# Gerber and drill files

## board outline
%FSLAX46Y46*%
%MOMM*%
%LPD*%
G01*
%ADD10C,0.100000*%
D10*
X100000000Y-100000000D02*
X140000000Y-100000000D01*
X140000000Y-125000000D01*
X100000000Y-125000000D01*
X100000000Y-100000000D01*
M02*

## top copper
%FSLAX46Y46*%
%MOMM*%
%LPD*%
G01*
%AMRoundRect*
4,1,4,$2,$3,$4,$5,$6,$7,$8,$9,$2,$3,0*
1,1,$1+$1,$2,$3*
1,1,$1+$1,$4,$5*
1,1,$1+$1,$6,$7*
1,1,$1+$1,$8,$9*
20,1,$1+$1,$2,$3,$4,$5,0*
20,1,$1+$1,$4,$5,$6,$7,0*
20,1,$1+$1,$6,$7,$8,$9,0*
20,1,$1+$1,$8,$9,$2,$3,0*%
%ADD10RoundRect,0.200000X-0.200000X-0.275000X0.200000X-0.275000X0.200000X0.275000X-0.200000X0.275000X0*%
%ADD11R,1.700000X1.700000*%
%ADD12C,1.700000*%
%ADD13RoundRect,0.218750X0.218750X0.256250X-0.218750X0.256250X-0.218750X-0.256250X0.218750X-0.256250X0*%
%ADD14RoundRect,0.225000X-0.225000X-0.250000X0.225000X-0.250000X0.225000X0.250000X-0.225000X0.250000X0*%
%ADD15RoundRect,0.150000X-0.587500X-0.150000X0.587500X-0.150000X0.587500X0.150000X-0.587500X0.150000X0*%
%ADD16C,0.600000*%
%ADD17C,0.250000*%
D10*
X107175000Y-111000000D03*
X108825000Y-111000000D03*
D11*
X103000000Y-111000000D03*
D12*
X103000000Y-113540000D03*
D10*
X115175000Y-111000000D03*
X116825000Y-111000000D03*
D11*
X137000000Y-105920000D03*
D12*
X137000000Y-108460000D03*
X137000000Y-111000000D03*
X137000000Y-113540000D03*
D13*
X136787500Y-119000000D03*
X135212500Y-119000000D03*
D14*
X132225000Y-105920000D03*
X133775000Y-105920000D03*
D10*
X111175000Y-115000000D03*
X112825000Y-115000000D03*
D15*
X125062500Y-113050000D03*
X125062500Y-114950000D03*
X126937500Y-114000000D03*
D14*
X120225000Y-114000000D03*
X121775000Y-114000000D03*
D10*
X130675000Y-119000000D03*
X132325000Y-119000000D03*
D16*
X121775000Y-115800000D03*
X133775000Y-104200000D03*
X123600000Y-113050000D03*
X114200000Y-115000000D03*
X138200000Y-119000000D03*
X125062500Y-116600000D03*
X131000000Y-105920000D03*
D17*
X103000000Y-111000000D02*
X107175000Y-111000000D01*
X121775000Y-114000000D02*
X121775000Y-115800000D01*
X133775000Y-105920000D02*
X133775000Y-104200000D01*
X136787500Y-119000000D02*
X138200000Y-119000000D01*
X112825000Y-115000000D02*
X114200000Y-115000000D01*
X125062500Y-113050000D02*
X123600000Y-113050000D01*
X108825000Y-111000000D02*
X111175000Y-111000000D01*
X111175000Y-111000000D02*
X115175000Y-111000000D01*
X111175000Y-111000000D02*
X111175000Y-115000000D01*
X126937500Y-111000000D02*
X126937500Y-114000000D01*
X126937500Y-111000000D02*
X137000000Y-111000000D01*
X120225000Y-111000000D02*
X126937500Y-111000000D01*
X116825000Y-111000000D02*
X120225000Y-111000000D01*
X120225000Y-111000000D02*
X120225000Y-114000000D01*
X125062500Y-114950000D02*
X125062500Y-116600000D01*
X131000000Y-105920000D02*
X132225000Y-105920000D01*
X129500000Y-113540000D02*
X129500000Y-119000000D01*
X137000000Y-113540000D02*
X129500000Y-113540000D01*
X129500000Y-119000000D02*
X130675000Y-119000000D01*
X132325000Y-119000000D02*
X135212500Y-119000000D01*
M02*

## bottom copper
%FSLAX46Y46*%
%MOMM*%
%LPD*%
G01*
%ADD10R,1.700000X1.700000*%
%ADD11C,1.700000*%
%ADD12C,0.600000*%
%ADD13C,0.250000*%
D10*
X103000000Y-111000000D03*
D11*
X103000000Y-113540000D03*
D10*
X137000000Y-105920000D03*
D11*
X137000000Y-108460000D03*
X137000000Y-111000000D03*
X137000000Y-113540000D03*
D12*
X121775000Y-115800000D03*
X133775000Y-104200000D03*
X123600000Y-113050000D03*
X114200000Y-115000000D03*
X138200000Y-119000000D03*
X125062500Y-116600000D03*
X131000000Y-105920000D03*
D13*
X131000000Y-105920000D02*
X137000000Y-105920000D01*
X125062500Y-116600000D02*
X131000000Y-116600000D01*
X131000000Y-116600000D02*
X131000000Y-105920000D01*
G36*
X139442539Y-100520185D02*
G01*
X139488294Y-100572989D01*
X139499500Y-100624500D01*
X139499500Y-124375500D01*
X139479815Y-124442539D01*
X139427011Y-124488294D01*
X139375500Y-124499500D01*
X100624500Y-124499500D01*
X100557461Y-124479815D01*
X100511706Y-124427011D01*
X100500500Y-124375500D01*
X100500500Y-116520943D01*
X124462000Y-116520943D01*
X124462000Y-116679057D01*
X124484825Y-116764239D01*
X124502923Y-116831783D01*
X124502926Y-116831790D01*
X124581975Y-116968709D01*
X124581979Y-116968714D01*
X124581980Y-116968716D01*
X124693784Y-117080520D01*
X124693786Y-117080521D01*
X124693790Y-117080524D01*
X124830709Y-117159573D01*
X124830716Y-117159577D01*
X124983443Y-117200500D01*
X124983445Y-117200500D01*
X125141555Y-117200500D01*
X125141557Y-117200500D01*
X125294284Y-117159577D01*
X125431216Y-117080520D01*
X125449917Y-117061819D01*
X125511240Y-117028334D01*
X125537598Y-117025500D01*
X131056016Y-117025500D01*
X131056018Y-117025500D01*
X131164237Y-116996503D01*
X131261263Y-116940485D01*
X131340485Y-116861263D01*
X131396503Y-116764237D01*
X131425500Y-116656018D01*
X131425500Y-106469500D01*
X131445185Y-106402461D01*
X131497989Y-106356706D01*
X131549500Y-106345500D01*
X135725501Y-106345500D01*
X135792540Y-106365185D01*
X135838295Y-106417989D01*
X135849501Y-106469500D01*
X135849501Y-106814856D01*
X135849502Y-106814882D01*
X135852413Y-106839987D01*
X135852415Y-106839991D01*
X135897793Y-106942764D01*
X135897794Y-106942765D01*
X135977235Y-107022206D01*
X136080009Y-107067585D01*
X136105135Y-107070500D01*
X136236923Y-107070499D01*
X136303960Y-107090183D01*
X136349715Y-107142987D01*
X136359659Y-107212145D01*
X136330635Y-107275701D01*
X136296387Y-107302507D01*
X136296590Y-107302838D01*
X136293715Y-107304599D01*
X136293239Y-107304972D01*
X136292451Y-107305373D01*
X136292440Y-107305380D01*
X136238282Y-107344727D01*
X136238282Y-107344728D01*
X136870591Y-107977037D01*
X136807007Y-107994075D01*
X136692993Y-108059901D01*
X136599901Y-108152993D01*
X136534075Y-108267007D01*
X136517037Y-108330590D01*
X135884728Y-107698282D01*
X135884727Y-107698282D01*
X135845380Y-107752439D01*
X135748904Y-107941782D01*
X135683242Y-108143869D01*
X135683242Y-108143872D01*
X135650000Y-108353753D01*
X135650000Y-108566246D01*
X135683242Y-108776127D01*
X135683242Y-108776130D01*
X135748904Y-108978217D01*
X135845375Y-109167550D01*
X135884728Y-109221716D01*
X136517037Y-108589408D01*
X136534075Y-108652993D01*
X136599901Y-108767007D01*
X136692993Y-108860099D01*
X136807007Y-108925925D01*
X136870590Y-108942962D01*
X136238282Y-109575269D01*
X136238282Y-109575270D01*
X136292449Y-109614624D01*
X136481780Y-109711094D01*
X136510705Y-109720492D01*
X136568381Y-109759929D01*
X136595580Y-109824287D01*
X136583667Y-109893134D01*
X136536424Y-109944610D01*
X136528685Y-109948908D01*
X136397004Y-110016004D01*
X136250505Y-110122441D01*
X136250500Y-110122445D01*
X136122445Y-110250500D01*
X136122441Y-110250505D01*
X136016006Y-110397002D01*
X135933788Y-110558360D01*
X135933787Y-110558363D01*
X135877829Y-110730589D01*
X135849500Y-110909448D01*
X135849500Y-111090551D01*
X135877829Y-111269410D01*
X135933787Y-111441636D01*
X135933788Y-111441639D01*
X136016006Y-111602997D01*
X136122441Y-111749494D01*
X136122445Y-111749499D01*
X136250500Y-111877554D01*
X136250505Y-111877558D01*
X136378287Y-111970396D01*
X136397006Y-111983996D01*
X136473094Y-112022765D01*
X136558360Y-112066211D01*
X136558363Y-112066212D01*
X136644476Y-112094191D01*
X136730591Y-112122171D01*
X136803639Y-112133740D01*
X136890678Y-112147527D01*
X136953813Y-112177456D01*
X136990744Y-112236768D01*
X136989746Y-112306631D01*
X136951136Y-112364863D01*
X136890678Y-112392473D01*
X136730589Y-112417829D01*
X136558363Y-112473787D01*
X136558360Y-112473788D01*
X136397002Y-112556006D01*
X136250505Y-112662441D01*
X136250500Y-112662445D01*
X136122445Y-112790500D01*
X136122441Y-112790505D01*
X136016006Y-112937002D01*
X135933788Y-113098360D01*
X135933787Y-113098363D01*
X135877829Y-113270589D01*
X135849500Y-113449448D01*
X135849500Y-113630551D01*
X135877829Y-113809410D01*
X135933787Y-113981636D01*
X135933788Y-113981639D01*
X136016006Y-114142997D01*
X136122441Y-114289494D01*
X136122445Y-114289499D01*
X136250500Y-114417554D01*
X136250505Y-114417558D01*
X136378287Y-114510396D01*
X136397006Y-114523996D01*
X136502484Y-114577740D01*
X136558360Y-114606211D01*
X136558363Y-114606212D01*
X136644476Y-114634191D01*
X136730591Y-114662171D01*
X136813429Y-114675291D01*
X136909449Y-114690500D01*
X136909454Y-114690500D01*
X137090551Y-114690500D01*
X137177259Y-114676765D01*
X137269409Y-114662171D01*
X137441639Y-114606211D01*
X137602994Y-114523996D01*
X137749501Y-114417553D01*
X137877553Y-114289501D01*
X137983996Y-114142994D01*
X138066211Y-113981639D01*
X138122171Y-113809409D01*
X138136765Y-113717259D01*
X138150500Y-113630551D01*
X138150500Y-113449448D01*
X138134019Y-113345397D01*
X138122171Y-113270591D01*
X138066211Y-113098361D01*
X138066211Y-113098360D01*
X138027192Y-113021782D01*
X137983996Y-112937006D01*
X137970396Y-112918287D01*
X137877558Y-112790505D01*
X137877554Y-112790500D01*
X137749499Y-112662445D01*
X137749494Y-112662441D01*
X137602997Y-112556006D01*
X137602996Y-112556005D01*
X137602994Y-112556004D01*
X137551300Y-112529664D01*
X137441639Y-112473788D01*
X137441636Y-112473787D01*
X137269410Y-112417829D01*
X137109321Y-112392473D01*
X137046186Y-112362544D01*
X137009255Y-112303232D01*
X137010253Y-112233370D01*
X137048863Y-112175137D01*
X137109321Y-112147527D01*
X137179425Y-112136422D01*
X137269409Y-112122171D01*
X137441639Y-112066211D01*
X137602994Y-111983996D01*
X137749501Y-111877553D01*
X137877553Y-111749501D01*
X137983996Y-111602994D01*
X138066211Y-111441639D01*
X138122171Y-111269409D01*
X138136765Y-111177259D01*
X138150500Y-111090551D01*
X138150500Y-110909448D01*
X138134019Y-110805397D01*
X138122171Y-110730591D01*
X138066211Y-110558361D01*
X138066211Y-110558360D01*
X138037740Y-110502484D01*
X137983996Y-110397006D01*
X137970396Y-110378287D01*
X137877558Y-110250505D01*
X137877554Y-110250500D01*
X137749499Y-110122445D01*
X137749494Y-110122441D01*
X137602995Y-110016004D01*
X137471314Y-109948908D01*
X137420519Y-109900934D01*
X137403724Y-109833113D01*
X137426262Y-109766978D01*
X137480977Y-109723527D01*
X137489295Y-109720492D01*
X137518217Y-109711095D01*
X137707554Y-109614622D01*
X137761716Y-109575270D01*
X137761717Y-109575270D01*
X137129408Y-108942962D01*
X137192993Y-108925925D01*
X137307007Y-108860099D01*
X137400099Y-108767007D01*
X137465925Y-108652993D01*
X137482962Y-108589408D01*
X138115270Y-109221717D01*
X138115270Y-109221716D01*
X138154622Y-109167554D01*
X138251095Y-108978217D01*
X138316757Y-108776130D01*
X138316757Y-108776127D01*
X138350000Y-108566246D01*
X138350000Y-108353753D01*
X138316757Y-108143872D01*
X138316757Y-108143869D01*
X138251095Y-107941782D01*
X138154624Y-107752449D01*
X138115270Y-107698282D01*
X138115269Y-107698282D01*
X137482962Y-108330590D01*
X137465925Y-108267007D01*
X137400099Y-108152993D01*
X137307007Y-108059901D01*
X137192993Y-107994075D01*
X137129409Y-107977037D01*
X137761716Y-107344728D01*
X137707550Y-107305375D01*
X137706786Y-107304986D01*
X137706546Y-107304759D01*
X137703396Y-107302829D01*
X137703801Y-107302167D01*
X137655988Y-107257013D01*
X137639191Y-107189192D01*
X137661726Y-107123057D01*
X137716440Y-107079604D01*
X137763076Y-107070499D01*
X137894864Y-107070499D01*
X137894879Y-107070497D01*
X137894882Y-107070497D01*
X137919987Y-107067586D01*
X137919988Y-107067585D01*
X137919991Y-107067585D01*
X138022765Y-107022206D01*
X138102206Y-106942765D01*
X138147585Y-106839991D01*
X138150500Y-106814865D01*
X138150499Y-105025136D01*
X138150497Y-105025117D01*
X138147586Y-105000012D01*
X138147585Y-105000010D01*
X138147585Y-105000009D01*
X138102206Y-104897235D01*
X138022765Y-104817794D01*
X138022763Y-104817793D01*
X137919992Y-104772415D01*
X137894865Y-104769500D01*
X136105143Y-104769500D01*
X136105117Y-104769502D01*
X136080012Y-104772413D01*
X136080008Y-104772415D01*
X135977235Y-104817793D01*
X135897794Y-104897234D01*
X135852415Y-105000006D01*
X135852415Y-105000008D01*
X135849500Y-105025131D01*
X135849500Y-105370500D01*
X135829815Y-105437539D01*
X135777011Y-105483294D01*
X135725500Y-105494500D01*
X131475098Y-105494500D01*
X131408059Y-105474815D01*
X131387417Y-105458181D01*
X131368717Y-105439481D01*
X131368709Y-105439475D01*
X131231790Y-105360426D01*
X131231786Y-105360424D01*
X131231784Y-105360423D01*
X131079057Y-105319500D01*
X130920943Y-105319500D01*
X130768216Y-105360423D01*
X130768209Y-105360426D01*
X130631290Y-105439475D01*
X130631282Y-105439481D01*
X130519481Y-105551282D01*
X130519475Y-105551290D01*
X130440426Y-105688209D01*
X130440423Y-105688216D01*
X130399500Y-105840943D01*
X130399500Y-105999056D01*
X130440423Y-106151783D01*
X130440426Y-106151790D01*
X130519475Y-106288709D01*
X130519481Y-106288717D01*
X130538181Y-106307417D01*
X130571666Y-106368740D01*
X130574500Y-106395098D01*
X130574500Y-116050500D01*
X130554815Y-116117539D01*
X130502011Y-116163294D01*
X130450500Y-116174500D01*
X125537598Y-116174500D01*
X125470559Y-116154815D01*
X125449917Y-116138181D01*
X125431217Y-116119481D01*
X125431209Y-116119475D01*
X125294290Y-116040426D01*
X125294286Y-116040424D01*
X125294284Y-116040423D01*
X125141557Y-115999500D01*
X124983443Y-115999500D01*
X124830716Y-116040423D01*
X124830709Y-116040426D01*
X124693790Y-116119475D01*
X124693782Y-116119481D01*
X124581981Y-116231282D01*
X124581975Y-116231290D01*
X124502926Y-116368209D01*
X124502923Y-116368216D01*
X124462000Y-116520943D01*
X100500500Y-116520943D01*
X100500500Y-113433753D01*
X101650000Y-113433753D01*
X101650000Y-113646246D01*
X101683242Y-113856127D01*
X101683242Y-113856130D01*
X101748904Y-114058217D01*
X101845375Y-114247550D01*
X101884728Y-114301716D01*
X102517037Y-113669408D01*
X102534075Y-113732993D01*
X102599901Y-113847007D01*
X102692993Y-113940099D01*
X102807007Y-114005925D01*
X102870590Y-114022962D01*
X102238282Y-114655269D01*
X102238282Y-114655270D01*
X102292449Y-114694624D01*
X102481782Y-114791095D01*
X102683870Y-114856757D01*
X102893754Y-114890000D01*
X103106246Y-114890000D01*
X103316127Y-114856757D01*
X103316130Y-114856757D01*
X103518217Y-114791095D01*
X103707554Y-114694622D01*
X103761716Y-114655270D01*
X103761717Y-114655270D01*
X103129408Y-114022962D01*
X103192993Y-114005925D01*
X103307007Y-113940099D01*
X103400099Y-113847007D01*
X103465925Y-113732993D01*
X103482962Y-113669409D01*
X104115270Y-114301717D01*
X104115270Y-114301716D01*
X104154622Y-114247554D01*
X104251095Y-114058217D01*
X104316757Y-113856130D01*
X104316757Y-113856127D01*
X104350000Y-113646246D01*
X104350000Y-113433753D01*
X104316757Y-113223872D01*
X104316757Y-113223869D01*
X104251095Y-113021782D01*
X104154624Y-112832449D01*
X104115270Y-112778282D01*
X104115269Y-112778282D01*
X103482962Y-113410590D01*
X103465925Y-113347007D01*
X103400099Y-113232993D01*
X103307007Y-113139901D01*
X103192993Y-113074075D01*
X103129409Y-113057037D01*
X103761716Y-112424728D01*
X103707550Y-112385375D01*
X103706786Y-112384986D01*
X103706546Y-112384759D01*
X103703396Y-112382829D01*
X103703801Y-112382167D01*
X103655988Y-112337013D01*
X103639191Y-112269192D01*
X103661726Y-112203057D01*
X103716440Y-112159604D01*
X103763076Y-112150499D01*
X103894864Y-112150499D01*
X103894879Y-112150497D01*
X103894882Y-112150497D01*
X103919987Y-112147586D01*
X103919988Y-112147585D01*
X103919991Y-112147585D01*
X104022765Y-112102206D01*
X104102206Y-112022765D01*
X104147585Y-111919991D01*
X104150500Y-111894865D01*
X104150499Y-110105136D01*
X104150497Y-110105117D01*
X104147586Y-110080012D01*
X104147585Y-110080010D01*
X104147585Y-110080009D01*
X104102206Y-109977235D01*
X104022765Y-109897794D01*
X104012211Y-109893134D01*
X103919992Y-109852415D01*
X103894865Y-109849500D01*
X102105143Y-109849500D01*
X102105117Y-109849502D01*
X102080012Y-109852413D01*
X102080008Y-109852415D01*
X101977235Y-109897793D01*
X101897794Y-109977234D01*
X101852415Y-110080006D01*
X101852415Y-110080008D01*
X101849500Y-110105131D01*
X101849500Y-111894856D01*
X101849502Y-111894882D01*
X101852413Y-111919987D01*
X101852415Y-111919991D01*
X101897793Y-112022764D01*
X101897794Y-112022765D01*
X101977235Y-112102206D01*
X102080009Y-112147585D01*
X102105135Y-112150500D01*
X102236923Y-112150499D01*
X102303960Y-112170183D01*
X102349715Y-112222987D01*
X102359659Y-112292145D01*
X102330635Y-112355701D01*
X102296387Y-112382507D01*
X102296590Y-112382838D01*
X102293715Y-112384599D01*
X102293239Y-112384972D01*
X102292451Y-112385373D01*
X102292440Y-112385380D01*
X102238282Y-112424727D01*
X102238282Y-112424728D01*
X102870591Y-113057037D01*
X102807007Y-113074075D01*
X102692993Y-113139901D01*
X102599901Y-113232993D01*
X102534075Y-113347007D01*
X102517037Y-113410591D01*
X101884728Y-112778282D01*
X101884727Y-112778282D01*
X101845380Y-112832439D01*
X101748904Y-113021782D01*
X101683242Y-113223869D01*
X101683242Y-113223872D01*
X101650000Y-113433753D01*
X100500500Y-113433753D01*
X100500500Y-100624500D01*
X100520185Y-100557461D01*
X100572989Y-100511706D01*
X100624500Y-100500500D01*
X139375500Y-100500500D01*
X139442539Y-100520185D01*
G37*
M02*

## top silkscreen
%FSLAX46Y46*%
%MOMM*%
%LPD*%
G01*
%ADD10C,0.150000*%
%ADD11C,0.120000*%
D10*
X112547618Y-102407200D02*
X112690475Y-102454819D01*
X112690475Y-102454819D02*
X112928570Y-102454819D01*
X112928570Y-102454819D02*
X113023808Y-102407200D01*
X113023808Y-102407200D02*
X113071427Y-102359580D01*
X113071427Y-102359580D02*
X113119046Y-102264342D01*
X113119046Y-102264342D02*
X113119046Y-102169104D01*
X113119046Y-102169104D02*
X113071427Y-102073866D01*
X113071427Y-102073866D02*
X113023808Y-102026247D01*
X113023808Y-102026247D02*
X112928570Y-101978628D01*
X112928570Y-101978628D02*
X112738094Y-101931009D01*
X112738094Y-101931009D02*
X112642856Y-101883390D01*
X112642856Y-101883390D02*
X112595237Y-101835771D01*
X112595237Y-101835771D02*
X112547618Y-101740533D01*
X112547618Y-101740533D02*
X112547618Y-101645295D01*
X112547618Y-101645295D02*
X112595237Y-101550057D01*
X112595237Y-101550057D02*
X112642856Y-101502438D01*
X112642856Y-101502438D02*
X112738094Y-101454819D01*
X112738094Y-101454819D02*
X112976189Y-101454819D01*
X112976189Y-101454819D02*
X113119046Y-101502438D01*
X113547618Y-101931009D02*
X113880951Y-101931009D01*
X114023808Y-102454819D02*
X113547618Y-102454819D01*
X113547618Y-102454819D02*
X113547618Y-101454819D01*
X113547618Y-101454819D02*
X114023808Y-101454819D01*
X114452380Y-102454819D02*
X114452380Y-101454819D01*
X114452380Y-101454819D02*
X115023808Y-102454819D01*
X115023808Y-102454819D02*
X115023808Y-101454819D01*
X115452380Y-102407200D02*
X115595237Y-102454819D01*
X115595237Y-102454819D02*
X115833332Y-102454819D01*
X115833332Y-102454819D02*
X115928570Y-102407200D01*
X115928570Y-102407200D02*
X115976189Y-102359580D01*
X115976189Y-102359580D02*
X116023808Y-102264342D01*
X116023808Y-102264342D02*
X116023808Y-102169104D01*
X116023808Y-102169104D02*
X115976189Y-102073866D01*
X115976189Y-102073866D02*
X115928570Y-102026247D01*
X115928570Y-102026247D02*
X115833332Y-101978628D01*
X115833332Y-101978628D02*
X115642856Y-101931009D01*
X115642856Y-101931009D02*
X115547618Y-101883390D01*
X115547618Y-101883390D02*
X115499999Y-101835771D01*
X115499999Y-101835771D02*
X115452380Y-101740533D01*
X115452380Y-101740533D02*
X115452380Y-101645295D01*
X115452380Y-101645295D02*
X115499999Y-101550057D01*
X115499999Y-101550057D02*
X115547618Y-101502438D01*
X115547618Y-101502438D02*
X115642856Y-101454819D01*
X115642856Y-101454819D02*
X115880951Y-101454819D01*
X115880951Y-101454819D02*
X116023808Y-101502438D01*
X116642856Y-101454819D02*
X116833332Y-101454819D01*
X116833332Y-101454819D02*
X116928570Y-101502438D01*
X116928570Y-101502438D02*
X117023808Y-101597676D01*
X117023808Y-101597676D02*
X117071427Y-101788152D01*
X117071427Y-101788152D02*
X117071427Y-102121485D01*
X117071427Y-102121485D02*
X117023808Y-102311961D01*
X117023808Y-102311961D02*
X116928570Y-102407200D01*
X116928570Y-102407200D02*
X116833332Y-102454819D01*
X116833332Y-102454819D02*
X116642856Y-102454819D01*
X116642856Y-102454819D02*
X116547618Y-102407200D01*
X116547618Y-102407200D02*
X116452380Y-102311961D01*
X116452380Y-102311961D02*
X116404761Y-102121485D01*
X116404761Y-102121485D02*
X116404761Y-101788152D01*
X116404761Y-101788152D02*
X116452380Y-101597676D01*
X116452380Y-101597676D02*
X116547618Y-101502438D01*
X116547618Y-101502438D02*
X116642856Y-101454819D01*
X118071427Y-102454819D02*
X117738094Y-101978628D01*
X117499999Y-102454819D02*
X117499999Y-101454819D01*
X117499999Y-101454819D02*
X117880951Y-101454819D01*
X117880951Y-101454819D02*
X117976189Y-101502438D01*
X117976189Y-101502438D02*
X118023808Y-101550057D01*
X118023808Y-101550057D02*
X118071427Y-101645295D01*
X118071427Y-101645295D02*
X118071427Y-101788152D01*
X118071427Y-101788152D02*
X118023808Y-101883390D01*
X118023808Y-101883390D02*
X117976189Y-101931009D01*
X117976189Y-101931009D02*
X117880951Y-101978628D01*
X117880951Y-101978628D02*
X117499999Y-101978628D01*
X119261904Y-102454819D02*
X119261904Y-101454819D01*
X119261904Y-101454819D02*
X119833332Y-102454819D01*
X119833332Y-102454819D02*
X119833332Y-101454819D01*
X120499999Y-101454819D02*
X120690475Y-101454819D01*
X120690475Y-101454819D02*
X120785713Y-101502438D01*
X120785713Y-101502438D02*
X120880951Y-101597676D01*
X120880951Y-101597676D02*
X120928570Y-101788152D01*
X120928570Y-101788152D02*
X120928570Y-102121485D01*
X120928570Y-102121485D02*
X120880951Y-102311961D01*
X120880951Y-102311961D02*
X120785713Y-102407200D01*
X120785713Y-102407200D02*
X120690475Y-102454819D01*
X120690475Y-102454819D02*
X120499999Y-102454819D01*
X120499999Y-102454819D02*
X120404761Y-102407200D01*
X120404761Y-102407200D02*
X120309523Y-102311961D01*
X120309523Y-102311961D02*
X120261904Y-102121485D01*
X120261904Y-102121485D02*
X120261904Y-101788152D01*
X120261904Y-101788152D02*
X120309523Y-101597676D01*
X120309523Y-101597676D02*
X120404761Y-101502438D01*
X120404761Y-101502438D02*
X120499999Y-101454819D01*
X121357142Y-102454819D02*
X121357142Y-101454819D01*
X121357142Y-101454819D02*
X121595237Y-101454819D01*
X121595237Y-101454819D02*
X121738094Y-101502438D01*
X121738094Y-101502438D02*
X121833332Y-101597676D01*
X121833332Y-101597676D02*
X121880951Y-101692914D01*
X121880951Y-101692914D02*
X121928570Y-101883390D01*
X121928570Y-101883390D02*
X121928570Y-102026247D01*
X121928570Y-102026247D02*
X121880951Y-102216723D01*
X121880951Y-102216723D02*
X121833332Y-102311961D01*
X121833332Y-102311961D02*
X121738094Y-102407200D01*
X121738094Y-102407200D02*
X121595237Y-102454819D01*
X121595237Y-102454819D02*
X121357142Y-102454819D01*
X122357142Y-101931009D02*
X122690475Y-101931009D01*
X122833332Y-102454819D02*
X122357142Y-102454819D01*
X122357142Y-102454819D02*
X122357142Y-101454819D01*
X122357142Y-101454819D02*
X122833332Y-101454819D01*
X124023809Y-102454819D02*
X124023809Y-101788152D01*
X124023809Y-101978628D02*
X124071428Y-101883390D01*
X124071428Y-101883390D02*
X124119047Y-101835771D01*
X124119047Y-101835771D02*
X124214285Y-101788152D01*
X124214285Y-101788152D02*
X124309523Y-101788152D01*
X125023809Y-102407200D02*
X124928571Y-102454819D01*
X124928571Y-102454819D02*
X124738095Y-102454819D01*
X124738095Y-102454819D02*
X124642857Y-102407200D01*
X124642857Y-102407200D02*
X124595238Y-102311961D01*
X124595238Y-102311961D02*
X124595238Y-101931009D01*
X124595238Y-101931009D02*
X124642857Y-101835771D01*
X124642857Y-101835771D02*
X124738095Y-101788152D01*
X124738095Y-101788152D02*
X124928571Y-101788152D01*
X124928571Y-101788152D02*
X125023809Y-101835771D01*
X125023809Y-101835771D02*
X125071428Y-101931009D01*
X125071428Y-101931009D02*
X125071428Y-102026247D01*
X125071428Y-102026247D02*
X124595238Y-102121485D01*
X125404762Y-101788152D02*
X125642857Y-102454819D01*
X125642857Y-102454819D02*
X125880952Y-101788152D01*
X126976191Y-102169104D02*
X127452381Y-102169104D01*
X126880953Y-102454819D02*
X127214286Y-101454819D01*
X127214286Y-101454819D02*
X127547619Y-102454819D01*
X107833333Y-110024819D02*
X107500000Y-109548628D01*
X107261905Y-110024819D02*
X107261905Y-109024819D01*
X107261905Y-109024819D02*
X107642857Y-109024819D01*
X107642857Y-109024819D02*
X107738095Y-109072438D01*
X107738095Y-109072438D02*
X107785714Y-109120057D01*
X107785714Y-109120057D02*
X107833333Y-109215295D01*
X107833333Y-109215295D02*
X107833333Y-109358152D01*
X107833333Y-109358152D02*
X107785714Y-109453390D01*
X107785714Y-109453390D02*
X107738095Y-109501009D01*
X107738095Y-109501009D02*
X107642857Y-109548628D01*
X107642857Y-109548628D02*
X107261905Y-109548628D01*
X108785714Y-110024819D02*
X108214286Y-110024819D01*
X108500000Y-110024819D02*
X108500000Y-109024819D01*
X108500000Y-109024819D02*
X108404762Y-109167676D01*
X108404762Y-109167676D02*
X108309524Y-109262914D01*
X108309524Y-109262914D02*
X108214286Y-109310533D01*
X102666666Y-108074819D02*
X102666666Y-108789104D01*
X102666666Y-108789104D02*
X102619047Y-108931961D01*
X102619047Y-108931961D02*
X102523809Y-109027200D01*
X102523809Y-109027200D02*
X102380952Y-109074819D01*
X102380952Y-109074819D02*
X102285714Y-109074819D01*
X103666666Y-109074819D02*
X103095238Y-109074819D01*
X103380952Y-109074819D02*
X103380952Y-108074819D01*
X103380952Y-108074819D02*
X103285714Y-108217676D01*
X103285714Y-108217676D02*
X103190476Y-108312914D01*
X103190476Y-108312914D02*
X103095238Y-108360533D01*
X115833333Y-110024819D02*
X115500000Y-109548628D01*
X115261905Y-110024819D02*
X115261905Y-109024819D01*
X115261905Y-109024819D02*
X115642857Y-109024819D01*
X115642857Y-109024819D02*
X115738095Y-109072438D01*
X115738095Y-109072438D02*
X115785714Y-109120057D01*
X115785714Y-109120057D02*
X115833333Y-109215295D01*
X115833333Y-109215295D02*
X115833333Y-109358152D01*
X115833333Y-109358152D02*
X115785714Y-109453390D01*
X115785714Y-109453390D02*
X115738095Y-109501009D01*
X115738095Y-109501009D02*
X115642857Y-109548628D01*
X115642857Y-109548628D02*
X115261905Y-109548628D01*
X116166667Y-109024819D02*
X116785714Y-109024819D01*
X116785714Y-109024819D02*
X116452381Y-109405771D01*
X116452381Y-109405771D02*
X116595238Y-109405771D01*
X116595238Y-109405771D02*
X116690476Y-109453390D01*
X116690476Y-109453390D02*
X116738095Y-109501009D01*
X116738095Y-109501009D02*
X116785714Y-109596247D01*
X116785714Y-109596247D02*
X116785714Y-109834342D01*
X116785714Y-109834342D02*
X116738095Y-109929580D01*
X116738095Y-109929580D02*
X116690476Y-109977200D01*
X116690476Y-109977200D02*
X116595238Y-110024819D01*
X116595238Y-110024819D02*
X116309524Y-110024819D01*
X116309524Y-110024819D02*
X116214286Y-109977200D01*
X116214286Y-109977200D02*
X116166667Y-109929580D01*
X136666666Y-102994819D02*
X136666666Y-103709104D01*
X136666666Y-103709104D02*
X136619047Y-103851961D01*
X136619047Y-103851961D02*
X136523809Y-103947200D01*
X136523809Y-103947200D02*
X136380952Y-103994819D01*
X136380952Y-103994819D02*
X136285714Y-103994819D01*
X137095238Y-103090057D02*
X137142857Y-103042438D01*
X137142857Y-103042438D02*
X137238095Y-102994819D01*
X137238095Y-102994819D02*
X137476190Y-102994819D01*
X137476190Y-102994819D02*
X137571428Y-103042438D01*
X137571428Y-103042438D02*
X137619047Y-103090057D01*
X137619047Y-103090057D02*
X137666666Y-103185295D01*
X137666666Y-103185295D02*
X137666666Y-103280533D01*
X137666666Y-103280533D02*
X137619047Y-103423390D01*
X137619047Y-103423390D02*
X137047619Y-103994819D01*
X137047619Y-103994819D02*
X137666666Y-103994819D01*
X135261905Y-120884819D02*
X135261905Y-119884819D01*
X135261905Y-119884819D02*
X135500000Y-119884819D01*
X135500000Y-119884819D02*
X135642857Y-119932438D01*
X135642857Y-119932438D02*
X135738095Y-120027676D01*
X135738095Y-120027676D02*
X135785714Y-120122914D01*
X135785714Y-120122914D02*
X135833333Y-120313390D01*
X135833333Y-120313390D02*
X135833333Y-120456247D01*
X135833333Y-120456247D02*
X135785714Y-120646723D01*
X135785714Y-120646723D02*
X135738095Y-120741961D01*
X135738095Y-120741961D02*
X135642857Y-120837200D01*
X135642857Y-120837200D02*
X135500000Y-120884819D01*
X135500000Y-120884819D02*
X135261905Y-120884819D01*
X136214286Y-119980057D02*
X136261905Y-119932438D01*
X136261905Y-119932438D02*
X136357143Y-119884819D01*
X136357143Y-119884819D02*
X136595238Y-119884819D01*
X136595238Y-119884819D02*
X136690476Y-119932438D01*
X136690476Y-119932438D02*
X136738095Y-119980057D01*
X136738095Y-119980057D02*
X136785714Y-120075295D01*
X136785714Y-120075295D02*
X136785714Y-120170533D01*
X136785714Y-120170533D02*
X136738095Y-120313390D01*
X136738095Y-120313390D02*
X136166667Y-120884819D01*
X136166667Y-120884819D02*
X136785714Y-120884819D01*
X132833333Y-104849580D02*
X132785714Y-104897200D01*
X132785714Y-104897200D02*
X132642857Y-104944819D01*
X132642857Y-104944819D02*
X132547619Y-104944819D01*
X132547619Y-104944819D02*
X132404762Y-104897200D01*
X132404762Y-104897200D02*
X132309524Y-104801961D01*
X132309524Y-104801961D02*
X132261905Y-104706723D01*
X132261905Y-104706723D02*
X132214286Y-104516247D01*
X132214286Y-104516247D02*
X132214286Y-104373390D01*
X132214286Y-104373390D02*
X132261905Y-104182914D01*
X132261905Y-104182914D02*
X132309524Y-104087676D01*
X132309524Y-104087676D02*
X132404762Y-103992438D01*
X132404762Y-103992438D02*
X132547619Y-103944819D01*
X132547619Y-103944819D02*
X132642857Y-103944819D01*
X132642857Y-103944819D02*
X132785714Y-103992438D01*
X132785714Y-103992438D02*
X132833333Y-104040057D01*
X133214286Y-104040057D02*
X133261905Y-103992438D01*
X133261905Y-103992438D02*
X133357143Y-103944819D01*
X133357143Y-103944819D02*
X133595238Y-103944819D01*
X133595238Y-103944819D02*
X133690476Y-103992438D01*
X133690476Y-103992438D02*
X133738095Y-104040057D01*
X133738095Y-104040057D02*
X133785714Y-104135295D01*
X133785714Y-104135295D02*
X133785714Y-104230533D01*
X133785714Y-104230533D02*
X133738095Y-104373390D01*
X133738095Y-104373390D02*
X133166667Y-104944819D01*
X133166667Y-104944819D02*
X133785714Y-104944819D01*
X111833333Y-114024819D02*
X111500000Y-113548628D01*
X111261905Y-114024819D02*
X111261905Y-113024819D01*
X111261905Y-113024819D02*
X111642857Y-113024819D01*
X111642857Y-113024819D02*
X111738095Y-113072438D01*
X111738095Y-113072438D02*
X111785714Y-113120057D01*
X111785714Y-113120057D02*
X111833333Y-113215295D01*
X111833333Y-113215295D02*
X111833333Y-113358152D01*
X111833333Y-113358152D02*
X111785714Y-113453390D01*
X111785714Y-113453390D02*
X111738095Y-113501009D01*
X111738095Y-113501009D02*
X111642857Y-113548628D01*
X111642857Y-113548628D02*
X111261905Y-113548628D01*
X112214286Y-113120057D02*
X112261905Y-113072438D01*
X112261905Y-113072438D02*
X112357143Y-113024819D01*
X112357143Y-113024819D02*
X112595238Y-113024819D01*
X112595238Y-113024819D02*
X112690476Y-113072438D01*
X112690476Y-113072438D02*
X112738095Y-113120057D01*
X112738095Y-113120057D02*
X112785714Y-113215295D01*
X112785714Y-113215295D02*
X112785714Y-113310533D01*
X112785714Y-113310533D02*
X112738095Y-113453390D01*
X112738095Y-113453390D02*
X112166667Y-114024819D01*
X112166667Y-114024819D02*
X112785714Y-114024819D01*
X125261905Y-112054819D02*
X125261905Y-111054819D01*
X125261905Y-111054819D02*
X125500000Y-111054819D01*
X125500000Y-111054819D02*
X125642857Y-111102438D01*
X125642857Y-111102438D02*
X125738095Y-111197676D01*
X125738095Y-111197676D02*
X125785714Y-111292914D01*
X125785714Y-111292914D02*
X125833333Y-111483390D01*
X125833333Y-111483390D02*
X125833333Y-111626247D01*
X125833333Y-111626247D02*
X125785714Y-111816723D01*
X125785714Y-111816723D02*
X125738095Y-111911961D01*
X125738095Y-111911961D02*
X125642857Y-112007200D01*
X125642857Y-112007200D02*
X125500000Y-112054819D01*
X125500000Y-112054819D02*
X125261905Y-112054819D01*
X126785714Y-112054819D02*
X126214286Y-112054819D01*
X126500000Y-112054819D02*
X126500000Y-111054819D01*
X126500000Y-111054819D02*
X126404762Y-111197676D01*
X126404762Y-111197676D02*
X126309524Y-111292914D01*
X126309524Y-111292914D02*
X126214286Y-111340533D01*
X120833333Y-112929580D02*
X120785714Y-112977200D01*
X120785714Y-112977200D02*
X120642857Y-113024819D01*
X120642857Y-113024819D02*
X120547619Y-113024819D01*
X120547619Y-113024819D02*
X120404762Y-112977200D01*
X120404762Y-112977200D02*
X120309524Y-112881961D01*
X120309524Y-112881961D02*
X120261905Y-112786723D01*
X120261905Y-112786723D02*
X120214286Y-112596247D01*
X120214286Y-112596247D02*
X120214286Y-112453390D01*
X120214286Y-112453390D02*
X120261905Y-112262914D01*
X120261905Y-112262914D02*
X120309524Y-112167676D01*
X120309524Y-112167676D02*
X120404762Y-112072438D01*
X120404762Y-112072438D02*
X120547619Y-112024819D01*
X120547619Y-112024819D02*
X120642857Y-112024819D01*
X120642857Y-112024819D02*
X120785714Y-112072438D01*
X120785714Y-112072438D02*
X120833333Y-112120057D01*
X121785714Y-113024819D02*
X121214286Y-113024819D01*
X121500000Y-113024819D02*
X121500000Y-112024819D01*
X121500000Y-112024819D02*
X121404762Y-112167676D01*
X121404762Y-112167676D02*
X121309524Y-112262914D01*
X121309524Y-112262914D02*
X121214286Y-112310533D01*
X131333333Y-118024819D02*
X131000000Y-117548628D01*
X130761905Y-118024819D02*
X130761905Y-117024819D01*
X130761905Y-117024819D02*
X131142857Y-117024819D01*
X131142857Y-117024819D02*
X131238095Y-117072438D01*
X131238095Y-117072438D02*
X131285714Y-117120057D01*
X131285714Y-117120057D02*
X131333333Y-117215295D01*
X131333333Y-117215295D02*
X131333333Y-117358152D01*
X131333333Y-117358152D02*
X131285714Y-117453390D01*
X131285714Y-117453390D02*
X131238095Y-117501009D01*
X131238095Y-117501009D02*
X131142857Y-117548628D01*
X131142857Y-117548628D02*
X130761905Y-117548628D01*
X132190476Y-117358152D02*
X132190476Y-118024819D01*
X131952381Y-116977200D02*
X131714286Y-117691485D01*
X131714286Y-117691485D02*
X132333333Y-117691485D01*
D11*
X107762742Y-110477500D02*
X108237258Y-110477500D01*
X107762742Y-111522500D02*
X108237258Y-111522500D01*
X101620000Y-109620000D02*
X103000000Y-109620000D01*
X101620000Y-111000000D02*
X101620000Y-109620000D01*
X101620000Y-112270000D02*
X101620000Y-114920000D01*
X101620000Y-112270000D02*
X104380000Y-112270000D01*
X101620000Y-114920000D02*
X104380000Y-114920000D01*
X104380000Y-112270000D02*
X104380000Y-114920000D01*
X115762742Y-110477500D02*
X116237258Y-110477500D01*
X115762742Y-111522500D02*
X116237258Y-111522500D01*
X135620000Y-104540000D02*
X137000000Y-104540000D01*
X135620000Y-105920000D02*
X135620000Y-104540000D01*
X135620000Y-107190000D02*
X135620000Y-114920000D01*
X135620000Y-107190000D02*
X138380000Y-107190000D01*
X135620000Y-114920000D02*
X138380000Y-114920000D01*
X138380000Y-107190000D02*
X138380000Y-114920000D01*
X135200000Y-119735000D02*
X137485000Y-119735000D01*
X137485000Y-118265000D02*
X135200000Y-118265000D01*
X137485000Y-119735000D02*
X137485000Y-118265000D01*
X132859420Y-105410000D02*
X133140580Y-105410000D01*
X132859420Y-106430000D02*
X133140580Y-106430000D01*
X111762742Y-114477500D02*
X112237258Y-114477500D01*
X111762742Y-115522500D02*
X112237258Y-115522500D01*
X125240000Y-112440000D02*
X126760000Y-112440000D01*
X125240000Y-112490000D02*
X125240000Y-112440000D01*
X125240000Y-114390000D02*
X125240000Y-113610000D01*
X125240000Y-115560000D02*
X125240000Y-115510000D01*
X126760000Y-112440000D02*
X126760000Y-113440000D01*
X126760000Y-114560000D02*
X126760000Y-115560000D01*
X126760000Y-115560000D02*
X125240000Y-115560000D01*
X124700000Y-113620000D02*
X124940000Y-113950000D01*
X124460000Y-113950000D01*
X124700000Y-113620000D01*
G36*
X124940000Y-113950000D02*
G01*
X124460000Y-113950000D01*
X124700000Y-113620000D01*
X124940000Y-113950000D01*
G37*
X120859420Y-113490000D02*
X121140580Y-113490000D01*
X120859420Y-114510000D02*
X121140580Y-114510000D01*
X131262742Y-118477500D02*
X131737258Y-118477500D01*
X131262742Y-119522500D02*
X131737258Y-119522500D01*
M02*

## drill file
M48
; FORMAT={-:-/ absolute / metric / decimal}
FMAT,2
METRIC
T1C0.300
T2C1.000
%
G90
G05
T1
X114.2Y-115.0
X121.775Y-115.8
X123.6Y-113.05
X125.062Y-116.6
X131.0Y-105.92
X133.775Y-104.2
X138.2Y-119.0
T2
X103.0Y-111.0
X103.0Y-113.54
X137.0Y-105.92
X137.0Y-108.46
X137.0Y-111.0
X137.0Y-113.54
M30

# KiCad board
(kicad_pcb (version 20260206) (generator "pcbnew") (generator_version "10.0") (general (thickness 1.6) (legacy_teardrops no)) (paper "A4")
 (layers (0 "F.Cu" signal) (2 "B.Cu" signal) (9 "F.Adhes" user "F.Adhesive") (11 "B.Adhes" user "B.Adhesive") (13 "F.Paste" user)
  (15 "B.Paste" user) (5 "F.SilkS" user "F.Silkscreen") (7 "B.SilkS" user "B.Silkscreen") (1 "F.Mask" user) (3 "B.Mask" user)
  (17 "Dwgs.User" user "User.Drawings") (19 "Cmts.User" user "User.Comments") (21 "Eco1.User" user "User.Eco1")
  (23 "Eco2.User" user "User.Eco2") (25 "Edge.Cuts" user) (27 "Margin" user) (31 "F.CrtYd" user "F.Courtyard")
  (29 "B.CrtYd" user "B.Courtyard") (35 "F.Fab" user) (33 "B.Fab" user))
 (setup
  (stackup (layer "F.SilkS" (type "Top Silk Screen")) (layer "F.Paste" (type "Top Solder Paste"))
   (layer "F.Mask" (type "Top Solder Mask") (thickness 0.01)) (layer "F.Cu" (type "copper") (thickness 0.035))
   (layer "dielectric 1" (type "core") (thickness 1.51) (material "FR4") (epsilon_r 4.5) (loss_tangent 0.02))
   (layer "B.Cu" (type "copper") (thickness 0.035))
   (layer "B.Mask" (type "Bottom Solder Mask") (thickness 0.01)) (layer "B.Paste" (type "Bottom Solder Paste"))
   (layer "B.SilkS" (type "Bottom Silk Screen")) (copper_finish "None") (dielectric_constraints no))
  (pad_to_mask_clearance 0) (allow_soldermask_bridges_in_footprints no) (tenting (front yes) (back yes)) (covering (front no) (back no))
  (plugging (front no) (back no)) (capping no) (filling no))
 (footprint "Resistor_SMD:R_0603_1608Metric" (layer "F.Cu") (at 108 111)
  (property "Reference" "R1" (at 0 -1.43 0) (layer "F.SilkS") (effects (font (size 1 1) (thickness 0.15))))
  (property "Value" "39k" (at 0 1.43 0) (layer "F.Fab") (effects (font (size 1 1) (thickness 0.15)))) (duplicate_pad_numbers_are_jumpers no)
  (fp_line (start -0.237258 -0.5225) (end 0.237258 -0.5225) (stroke (width 0.12) (type solid)) (layer "F.SilkS"))
  (fp_line (start -0.237258 0.5225) (end 0.237258 0.5225) (stroke (width 0.12) (type solid)) (layer "F.SilkS"))
  (pad "1" smd roundrect (at -0.825 0) (size 0.8 0.95) (layers "F.Cu" "F.Mask" "F.Paste") (roundrect_rratio 0.25) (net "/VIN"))
  (pad "2" smd roundrect (at 0.825 0) (size 0.8 0.95) (layers "F.Cu" "F.Mask" "F.Paste") (roundrect_rratio 0.25) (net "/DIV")))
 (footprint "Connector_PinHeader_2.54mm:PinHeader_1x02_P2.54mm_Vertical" (layer "F.Cu") (at 103 111)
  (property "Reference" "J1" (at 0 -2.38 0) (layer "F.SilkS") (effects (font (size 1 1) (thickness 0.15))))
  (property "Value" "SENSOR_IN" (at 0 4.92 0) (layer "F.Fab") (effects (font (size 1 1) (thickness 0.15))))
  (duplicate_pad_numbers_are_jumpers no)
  (fp_line (start -1.38 -1.38) (end 0 -1.38) (stroke (width 0.12) (type solid)) (layer "F.SilkS"))
  (fp_line (start -1.38 0) (end -1.38 -1.38) (stroke (width 0.12) (type solid)) (layer "F.SilkS"))
  (fp_line (start -1.38 1.27) (end -1.38 3.92) (stroke (width 0.12) (type solid)) (layer "F.SilkS"))
  (fp_line (start -1.38 1.27) (end 1.38 1.27) (stroke (width 0.12) (type solid)) (layer "F.SilkS"))
  (fp_line (start -1.38 3.92) (end 1.38 3.92) (stroke (width 0.12) (type solid)) (layer "F.SilkS"))
  (fp_line (start 1.38 1.27) (end 1.38 3.92) (stroke (width 0.12) (type solid)) (layer "F.SilkS"))
  (pad "1" thru_hole rect (at 0 0) (size 1.7 1.7) (drill 1) (layers "*.Cu" "*.Mask") (remove_unused_layers no) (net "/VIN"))
  (pad "2" thru_hole circle (at 0 2.54) (size 1.7 1.7) (drill 1) (layers "*.Cu" "*.Mask") (remove_unused_layers no) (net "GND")))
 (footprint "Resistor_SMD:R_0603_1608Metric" (layer "F.Cu") (at 116 111)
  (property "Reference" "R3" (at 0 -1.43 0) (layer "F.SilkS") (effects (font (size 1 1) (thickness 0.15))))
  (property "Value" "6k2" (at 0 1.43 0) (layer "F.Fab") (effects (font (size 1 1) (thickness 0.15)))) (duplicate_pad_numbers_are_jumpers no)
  (fp_line (start -0.237258 -0.5225) (end 0.237258 -0.5225) (stroke (width 0.12) (type solid)) (layer "F.SilkS"))
  (fp_line (start -0.237258 0.5225) (end 0.237258 0.5225) (stroke (width 0.12) (type solid)) (layer "F.SilkS"))
  (pad "1" smd roundrect (at -0.825 0) (size 0.8 0.95) (layers "F.Cu" "F.Mask" "F.Paste") (roundrect_rratio 0.25) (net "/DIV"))
  (pad "2" smd roundrect (at 0.825 0) (size 0.8 0.95) (layers "F.Cu" "F.Mask" "F.Paste") (roundrect_rratio 0.25) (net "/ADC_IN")))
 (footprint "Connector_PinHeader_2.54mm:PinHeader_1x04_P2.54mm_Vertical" (layer "F.Cu") (at 137 105.92)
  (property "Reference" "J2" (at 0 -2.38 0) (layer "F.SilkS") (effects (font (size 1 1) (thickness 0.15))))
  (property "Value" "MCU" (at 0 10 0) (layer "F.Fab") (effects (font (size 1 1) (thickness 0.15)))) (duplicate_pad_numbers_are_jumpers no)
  (fp_line (start -1.38 -1.38) (end 0 -1.38) (stroke (width 0.12) (type solid)) (layer "F.SilkS"))
  (fp_line (start -1.38 0) (end -1.38 -1.38) (stroke (width 0.12) (type solid)) (layer "F.SilkS"))
  (fp_line (start -1.38 1.27) (end -1.38 9) (stroke (width 0.12) (type solid)) (layer "F.SilkS"))
  (fp_line (start -1.38 1.27) (end 1.38 1.27) (stroke (width 0.12) (type solid)) (layer "F.SilkS"))
  (fp_line (start -1.38 9) (end 1.38 9) (stroke (width 0.12) (type solid)) (layer "F.SilkS"))
  (fp_line (start 1.38 1.27) (end 1.38 9) (stroke (width 0.12) (type solid)) (layer "F.SilkS"))
  (pad "1" thru_hole rect (at 0 0) (size 1.7 1.7) (drill 1) (layers "*.Cu" "*.Mask") (remove_unused_layers no) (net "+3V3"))
  (pad "2" thru_hole circle (at 0 2.54) (size 1.7 1.7) (drill 1) (layers "*.Cu" "*.Mask") (remove_unused_layers no) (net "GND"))
  (pad "3" thru_hole circle (at 0 5.08) (size 1.7 1.7) (drill 1) (layers "*.Cu" "*.Mask") (remove_unused_layers no) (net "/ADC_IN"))
  (pad "4" thru_hole circle (at 0 7.62) (size 1.7 1.7) (drill 1) (layers "*.Cu" "*.Mask") (remove_unused_layers no) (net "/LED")))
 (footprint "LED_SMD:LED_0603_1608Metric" (layer "F.Cu") (at 136 119 180)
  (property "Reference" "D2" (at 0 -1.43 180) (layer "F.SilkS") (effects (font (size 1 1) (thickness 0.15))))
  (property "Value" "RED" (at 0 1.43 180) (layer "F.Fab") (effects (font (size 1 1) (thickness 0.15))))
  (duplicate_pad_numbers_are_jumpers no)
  (fp_line (start 0.8 -0.735) (end -1.485 -0.735) (stroke (width 0.12) (type solid)) (layer "F.SilkS"))
  (fp_line (start -1.485 0.735) (end 0.8 0.735) (stroke (width 0.12) (type solid)) (layer "F.SilkS"))
  (fp_line (start -1.485 -0.735) (end -1.485 0.735) (stroke (width 0.12) (type solid)) (layer "F.SilkS"))
  (pad "1" smd roundrect (at -0.7875 0 180) (size 0.875 0.95) (layers "F.Cu" "F.Mask" "F.Paste") (roundrect_rratio 0.25) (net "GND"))
  (pad "2" smd roundrect (at 0.7875 0 180) (size 0.875 0.95) (layers "F.Cu" "F.Mask" "F.Paste") (roundrect_rratio 0.25) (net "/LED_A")))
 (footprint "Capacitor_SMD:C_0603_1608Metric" (layer "F.Cu") (at 133 105.92)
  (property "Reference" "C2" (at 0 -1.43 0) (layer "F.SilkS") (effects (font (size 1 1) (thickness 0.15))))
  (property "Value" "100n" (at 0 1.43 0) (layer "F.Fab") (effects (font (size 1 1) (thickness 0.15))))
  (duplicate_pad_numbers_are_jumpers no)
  (fp_line (start -0.14058 -0.51) (end 0.14058 -0.51) (stroke (width 0.12) (type solid)) (layer "F.SilkS"))
  (fp_line (start -0.14058 0.51) (end 0.14058 0.51) (stroke (width 0.12) (type solid)) (layer "F.SilkS"))
  (pad "1" smd roundrect (at -0.775 0) (size 0.9 0.95) (layers "F.Cu" "F.Mask" "F.Paste") (roundrect_rratio 0.25) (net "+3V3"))
  (pad "2" smd roundrect (at 0.775 0) (size 0.9 0.95) (layers "F.Cu" "F.Mask" "F.Paste") (roundrect_rratio 0.25) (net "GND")))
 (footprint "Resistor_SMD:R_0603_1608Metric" (layer "F.Cu") (at 112 115)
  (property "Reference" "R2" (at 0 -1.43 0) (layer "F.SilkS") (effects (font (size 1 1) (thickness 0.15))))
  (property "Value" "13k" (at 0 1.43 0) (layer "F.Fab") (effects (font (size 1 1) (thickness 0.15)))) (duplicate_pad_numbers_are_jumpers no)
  (fp_line (start -0.237258 -0.5225) (end 0.237258 -0.5225) (stroke (width 0.12) (type solid)) (layer "F.SilkS"))
  (fp_line (start -0.237258 0.5225) (end 0.237258 0.5225) (stroke (width 0.12) (type solid)) (layer "F.SilkS"))
  (pad "1" smd roundrect (at -0.825 0) (size 0.8 0.95) (layers "F.Cu" "F.Mask" "F.Paste") (roundrect_rratio 0.25) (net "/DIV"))
  (pad "2" smd roundrect (at 0.825 0) (size 0.8 0.95) (layers "F.Cu" "F.Mask" "F.Paste") (roundrect_rratio 0.25) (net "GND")))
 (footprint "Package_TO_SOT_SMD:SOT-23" (layer "F.Cu") (at 126 114)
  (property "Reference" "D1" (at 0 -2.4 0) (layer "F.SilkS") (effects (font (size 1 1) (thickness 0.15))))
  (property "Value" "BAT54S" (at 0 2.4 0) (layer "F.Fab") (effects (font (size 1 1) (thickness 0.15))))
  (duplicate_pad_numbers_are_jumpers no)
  (fp_line (start -0.76 -1.56) (end 0.76 -1.56) (stroke (width 0.12) (type solid)) (layer "F.SilkS"))
  (fp_line (start -0.76 -1.51) (end -0.76 -1.56) (stroke (width 0.12) (type solid)) (layer "F.SilkS"))
  (fp_line (start -0.76 0.39) (end -0.76 -0.39) (stroke (width 0.12) (type solid)) (layer "F.SilkS"))
  (fp_line (start -0.76 1.56) (end -0.76 1.51) (stroke (width 0.12) (type solid)) (layer "F.SilkS"))
  (fp_line (start 0.76 -1.56) (end 0.76 -0.56) (stroke (width 0.12) (type solid)) (layer "F.SilkS"))
  (fp_line (start 0.76 0.56) (end 0.76 1.56) (stroke (width 0.12) (type solid)) (layer "F.SilkS"))
  (fp_line (start 0.76 1.56) (end -0.76 1.56) (stroke (width 0.12) (type solid)) (layer "F.SilkS"))
  (fp_poly (pts (xy -1.3 -0.38) (xy -1.06 -0.05) (xy -1.54 -0.05)) (stroke (width 0.12) (type solid)) (fill yes) (layer "F.SilkS"))
  (pad "1" smd roundrect (at -0.9375 -0.95) (size 1.475 0.6) (layers "F.Cu" "F.Mask" "F.Paste") (roundrect_rratio 0.25) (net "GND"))
  (pad "2" smd roundrect (at -0.9375 0.95) (size 1.475 0.6) (layers "F.Cu" "F.Mask" "F.Paste") (roundrect_rratio 0.25) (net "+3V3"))
  (pad "3" smd roundrect (at 0.9375 0) (size 1.475 0.6) (layers "F.Cu" "F.Mask" "F.Paste") (roundrect_rratio 0.25) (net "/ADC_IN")))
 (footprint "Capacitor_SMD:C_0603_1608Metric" (layer "F.Cu") (at 121 114)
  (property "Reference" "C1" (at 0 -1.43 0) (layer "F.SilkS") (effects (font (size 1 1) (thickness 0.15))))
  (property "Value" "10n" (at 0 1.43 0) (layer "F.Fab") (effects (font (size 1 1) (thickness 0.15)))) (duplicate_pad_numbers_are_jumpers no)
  (fp_line (start -0.14058 -0.51) (end 0.14058 -0.51) (stroke (width 0.12) (type solid)) (layer "F.SilkS"))
  (fp_line (start -0.14058 0.51) (end 0.14058 0.51) (stroke (width 0.12) (type solid)) (layer "F.SilkS"))
  (pad "1" smd roundrect (at -0.775 0) (size 0.9 0.95) (layers "F.Cu" "F.Mask" "F.Paste") (roundrect_rratio 0.25) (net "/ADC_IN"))
  (pad "2" smd roundrect (at 0.775 0) (size 0.9 0.95) (layers "F.Cu" "F.Mask" "F.Paste") (roundrect_rratio 0.25) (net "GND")))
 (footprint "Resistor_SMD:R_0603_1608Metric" (layer "F.Cu") (at 131.5 119)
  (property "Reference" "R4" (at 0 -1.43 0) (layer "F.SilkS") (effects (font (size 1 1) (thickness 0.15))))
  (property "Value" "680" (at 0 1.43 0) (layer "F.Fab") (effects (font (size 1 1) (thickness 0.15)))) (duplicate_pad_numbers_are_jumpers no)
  (fp_line (start -0.237258 -0.5225) (end 0.237258 -0.5225) (stroke (width 0.12) (type solid)) (layer "F.SilkS"))
  (fp_line (start -0.237258 0.5225) (end 0.237258 0.5225) (stroke (width 0.12) (type solid)) (layer "F.SilkS"))
  (pad "1" smd roundrect (at -0.825 0) (size 0.8 0.95) (layers "F.Cu" "F.Mask" "F.Paste") (roundrect_rratio 0.25) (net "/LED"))
  (pad "2" smd roundrect (at 0.825 0) (size 0.8 0.95) (layers "F.Cu" "F.Mask" "F.Paste") (roundrect_rratio 0.25) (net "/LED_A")))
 (gr_rect (start 100 100) (end 140 125) (stroke (width 0.1) (type default)) (fill no) (layer "Edge.Cuts"))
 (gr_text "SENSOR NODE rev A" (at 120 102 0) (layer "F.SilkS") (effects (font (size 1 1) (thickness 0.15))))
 (segment (start 103 111) (end 107.175 111) (width 0.25) (layer "F.Cu") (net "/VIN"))
 (segment (start 121.775 114) (end 121.775 115.8) (width 0.25) (layer "F.Cu") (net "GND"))
 (segment (start 133.775 105.92) (end 133.775 104.2) (width 0.25) (layer "F.Cu") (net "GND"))
 (segment (start 136.7875 119) (end 138.2 119) (width 0.25) (layer "F.Cu") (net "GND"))
 (segment (start 112.825 115) (end 114.2 115) (width 0.25) (layer "F.Cu") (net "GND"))
 (segment (start 125.0625 113.05) (end 123.6 113.05) (width 0.25) (layer "F.Cu") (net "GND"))
 (via (at 121.775 115.8) (size 0.6) (drill 0.3) (layers "F.Cu" "B.Cu") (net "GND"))
 (via (at 133.775 104.2) (size 0.6) (drill 0.3) (layers "F.Cu" "B.Cu") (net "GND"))
 (via (at 123.6 113.05) (size 0.6) (drill 0.3) (layers "F.Cu" "B.Cu") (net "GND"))
 (via (at 114.2 115) (size 0.6) (drill 0.3) (layers "F.Cu" "B.Cu") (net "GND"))
 (via (at 138.2 119) (size 0.6) (drill 0.3) (layers "F.Cu" "B.Cu") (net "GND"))
 (segment (start 108.825 111) (end 111.175 111) (width 0.25) (layer "F.Cu") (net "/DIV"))
 (segment (start 111.175 111) (end 115.175 111) (width 0.25) (layer "F.Cu") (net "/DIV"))
 (segment (start 111.175 111) (end 111.175 115) (width 0.25) (layer "F.Cu") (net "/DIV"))
 (segment (start 126.9375 111) (end 126.9375 114) (width 0.25) (layer "F.Cu") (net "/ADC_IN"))
 (segment (start 126.9375 111) (end 137 111) (width 0.25) (layer "F.Cu") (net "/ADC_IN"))
 (segment (start 120.225 111) (end 126.9375 111) (width 0.25) (layer "F.Cu") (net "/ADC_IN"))
 (segment (start 116.825 111) (end 120.225 111) (width 0.25) (layer "F.Cu") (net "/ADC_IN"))
 (segment (start 120.225 111) (end 120.225 114) (width 0.25) (layer "F.Cu") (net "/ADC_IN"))
 (segment (start 125.0625 114.95) (end 125.0625 116.6) (width 0.25) (layer "F.Cu") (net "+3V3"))
 (segment (start 131 105.92) (end 132.225 105.92) (width 0.25) (layer "F.Cu") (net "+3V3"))
 (via (at 125.0625 116.6) (size 0.6) (drill 0.3) (layers "F.Cu" "B.Cu") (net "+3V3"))
 (via (at 131 105.92) (size 0.6) (drill 0.3) (layers "F.Cu" "B.Cu") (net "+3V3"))
 (segment (start 131 105.92) (end 137 105.92) (width 0.25) (layer "B.Cu") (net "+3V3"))
 (segment (start 125.0625 116.6) (end 131 116.6) (width 0.25) (layer "B.Cu") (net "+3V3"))
 (segment (start 131 116.6) (end 131 105.92) (width 0.25) (layer "B.Cu") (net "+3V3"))
 (segment (start 129.5 113.54) (end 129.5 119) (width 0.25) (layer "F.Cu") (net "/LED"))
 (segment (start 137 113.54) (end 129.5 113.54) (width 0.25) (layer "F.Cu") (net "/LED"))
 (segment (start 129.5 119) (end 130.675 119) (width 0.25) (layer "F.Cu") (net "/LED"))
 (segment (start 132.325 119) (end 135.2125 119) (width 0.25) (layer "F.Cu") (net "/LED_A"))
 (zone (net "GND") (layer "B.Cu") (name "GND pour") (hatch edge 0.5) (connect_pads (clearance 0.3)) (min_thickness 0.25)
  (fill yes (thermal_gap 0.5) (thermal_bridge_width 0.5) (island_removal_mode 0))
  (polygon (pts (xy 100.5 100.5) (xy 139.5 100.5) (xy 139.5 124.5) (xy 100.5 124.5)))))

